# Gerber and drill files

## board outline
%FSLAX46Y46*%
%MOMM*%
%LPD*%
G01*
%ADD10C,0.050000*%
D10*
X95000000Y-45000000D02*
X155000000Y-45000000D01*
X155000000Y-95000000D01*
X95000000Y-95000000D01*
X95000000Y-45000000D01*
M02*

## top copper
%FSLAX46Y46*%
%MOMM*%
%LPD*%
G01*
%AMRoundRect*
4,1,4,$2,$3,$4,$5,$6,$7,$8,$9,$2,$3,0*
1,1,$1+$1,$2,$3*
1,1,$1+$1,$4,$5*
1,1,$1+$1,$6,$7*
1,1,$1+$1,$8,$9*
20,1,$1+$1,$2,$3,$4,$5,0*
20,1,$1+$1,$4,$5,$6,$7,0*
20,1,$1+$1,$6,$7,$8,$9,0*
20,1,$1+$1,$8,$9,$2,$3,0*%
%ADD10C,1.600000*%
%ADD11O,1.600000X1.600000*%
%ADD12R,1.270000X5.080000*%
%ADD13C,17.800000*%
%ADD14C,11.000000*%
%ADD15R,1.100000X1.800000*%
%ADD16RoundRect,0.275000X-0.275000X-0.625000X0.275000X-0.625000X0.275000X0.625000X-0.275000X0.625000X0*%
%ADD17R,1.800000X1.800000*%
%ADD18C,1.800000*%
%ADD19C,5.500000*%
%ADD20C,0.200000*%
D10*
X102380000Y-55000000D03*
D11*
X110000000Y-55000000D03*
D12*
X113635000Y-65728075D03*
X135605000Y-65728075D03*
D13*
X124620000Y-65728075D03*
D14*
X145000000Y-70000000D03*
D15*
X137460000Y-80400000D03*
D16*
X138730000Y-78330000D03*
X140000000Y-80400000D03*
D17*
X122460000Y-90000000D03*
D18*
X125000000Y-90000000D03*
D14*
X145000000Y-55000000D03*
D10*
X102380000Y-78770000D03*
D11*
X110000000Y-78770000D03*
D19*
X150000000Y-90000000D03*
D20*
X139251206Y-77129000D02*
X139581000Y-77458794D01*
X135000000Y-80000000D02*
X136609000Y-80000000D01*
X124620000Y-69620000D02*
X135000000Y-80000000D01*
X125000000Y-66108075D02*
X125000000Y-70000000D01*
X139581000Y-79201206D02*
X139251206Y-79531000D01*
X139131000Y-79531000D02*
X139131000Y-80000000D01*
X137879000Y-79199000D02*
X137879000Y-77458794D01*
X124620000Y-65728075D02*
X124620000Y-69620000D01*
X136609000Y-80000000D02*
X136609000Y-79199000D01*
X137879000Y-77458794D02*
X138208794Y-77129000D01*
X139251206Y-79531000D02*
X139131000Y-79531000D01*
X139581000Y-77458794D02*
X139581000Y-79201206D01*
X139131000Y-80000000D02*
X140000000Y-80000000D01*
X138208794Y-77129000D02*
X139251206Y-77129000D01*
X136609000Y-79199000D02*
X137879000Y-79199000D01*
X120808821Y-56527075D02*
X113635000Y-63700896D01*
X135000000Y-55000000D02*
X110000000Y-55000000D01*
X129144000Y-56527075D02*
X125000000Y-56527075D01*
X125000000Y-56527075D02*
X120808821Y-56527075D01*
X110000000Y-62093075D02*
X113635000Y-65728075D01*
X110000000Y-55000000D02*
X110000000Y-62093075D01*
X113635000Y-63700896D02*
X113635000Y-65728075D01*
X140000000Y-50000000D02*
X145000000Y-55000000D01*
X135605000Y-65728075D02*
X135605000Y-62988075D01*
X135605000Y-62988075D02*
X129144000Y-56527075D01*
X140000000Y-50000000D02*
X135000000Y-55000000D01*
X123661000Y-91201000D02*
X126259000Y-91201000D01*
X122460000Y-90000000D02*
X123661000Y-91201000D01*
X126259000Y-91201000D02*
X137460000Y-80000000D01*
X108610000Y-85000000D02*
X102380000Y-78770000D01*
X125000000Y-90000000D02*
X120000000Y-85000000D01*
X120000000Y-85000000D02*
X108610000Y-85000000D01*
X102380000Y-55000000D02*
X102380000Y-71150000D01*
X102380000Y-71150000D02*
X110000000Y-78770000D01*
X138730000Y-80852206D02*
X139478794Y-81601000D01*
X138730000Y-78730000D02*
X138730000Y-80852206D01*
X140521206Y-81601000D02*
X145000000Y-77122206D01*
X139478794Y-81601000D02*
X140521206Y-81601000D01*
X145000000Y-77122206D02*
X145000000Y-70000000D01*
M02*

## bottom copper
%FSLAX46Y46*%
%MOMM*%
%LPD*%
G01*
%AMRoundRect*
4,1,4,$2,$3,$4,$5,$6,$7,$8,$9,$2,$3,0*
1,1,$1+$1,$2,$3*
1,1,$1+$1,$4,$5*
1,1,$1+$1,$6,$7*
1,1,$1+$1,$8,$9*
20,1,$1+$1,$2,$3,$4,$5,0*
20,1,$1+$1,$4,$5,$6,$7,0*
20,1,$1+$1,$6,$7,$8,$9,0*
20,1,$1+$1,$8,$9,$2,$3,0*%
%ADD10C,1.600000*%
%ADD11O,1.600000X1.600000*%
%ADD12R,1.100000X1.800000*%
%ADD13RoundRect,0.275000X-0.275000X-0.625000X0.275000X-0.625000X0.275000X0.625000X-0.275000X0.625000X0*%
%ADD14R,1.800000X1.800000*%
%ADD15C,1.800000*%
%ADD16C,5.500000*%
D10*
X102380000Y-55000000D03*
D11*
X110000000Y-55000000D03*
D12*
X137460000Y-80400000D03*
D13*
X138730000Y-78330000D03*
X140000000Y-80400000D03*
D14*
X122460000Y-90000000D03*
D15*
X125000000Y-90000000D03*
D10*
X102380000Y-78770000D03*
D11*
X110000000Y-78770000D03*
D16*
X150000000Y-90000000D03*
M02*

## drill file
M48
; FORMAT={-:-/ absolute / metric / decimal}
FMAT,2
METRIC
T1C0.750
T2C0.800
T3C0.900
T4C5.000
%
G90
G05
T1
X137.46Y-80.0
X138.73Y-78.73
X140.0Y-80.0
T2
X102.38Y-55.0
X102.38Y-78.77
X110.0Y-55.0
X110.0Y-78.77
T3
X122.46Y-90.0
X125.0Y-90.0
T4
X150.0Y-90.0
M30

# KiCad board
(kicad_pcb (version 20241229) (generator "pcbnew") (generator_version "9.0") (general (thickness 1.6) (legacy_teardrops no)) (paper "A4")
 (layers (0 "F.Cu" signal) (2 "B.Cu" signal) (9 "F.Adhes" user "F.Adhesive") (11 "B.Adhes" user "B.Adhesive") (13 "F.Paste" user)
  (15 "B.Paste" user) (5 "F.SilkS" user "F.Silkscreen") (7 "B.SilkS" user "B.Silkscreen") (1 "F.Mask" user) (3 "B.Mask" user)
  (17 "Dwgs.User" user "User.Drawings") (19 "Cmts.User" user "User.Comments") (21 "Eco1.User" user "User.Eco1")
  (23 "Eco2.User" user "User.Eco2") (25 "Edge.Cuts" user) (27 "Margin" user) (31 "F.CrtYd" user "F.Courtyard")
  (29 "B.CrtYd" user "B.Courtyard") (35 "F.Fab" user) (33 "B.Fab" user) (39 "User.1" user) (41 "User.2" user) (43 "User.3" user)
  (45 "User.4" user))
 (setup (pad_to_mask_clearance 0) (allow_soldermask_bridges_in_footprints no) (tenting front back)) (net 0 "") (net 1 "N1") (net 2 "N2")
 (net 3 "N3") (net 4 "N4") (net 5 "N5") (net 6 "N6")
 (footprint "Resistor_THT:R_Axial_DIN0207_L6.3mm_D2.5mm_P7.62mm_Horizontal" (layer "F.Cu") (at 102.38 55)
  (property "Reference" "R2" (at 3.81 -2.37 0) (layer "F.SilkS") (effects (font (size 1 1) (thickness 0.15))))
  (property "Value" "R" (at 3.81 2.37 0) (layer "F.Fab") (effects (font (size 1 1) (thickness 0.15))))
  (pad "1" thru_hole circle (at 0 0) (size 1.6 1.6) (drill 0.8) (layers "*.Cu" "*.Mask") (remove_unused_layers no) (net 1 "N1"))
  (pad "2" thru_hole oval (at 7.62 0) (size 1.6 1.6) (drill 0.8) (layers "*.Cu" "*.Mask") (remove_unused_layers no) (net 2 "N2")))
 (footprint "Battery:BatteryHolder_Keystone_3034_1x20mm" (layer "F.Cu") (at 124.62 65.728075)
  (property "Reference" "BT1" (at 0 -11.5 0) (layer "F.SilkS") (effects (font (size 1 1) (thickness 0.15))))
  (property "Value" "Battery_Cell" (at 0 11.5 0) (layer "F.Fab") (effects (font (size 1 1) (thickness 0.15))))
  (pad "1" smd rect (at -10.985 0) (size 1.27 5.08) (layers "F.Cu" "F.Mask" "F.Paste") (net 2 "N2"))
  (pad "1" smd rect (at 10.985 0) (size 1.27 5.08) (layers "F.Cu" "F.Mask" "F.Paste") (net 2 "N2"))
  (pad "2" smd circle (at 0 0) (size 17.8 17.8) (layers "F.Cu" "F.Mask") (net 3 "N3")))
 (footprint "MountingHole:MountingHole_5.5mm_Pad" (layer "F.Cu") (at 145 70)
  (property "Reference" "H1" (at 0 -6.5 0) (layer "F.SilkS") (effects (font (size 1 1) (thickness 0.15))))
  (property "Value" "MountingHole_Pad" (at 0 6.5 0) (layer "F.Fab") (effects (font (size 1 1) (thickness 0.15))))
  (pad "1" smd circle (at 0 0) (size 11 11) (layers "F.Cu" "F.Mask" "F.Paste") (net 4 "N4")))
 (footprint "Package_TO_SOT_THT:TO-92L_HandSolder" (layer "F.Cu") (at 137.46 80)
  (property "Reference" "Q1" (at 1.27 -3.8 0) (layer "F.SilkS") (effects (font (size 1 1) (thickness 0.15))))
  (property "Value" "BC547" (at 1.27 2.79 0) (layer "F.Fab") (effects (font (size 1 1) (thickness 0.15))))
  (pad "1" thru_hole rect (at 0 0) (size 1.1 1.8) (drill 0.75 (offset 0 0.4)) (layers "*.Cu" "*.Mask") (remove_unused_layers no)
   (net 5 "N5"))
  (pad "2" thru_hole roundrect (at 1.27 -1.27) (size 1.1 1.8) (drill 0.75 (offset 0 -0.4)) (layers "*.Cu" "*.Mask")
   (remove_unused_layers no) (roundrect_rratio 0.25) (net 4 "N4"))
  (pad "3" thru_hole roundrect (at 2.54 0) (size 1.1 1.8) (drill 0.75 (offset 0 0.4)) (layers "*.Cu" "*.Mask") (remove_unused_layers no)
   (roundrect_rratio 0.25) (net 3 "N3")))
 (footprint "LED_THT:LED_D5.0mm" (layer "F.Cu") (at 122.46 90)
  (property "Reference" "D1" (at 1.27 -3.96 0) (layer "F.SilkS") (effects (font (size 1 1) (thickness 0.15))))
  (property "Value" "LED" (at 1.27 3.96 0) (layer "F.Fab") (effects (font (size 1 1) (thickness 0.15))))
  (pad "1" thru_hole rect (at 0 0) (size 1.8 1.8) (drill 0.9) (layers "*.Cu" "*.Mask") (remove_unused_layers no) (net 5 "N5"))
  (pad "2" thru_hole circle (at 2.54 0) (size 1.8 1.8) (drill 0.9) (layers "*.Cu" "*.Mask") (remove_unused_layers no) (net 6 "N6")))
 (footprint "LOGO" (layer "F.Cu") (at 140 90)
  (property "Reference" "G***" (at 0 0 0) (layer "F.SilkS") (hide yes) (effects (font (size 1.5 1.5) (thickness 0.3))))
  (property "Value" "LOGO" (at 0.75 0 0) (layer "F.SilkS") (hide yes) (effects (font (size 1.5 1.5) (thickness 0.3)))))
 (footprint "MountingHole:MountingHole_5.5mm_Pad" (layer "F.Cu") (at 145 55)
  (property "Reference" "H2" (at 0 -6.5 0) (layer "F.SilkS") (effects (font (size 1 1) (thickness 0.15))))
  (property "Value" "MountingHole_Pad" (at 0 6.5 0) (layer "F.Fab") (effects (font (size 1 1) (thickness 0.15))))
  (pad "1" smd circle (at 0 0) (size 11 11) (layers "F.Cu" "F.Mask" "F.Paste") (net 2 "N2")))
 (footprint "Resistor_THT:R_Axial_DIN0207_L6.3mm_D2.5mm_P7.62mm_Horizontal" (layer "F.Cu") (at 102.38 78.77)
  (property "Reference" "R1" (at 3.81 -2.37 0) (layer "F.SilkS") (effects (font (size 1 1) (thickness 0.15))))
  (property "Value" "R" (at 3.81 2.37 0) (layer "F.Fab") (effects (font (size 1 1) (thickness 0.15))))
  (pad "1" thru_hole circle (at 0 0) (size 1.6 1.6) (drill 0.8) (layers "*.Cu" "*.Mask") (remove_unused_layers no) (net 6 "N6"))
  (pad "2" thru_hole oval (at 7.62 0) (size 1.6 1.6) (drill 0.8) (layers "*.Cu" "*.Mask") (remove_unused_layers no) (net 1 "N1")))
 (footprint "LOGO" (layer "F.Cu") (at 101.514924 88.465482)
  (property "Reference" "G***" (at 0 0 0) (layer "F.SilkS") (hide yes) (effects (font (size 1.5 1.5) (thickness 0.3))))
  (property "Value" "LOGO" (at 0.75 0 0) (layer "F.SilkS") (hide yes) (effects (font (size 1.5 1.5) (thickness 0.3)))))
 (gr_poly (pts (xy 95 45) (xy 155 45) (xy 155 95) (xy 95 95)) (stroke (width 0.05) (type solid)) (fill no) (locked yes) (layer "Edge.Cuts"))
 (via (at 150 90) (size 5.5) (drill 5) (layers "F.Cu" "B.Cu") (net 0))
 (segment (start 139.251206 77.129) (end 139.581 77.458794) (width 0.2) (layer "F.Cu") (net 3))
 (segment (start 135 80) (end 136.609 80) (width 0.2) (layer "F.Cu") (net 3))
 (segment (start 124.62 69.62) (end 135 80) (width 0.2) (layer "F.Cu") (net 3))
 (segment (start 125 66.108075) (end 125 70) (width 0.2) (layer "F.Cu") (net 3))
 (segment (start 139.581 79.201206) (end 139.251206 79.531) (width 0.2) (layer "F.Cu") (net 3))
 (segment (start 139.131 79.531) (end 139.131 80) (width 0.2) (layer "F.Cu") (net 3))
 (segment (start 137.879 79.199) (end 137.879 77.458794) (width 0.2) (layer "F.Cu") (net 3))
 (segment (start 124.62 65.728075) (end 124.62 69.62) (width 0.2) (layer "F.Cu") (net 3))
 (segment (start 136.609 80) (end 136.609 79.199) (width 0.2) (layer "F.Cu") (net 3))
 (segment (start 137.879 77.458794) (end 138.208794 77.129) (width 0.2) (layer "F.Cu") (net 3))
 (segment (start 139.251206 79.531) (end 139.131 79.531) (width 0.2) (layer "F.Cu") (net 3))
 (segment (start 139.581 77.458794) (end 139.581 79.201206) (width 0.2) (layer "F.Cu") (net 3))
 (segment (start 139.131 80) (end 140 80) (width 0.2) (layer "F.Cu") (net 3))
 (segment (start 138.208794 77.129) (end 139.251206 77.129) (width 0.2) (layer "F.Cu") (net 3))
 (segment (start 136.609 79.199) (end 137.879 79.199) (width 0.2) (layer "F.Cu") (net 3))
 (segment (start 120.808821 56.527075) (end 113.635 63.700896) (width 0.2) (layer "F.Cu") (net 2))
 (segment (start 135 55) (end 110 55) (width 0.2) (layer "F.Cu") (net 2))
 (segment (start 129.144 56.527075) (end 125 56.527075) (width 0.2) (layer "F.Cu") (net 2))
 (segment (start 125 56.527075) (end 120.808821 56.527075) (width 0.2) (layer "F.Cu") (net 2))
 (segment (start 110 62.093075) (end 113.635 65.728075) (width 0.2) (layer "F.Cu") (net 2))
 (segment (start 110 55) (end 110 62.093075) (width 0.2) (layer "F.Cu") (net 2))
 (segment (start 113.635 63.700896) (end 113.635 65.728075) (width 0.2) (layer "F.Cu") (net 2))
 (segment (start 140 50) (end 145 55) (width 0.2) (layer "F.Cu") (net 2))
 (segment (start 135.605 65.728075) (end 135.605 62.988075) (width 0.2) (layer "F.Cu") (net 2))
 (segment (start 135.605 62.988075) (end 129.144 56.527075) (width 0.2) (layer "F.Cu") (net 2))
 (segment (start 140 50) (end 135 55) (width 0.2) (layer "F.Cu") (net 2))
 (segment (start 123.661 91.201) (end 126.259 91.201) (width 0.2) (layer "F.Cu") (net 5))
 (segment (start 122.46 90) (end 123.661 91.201) (width 0.2) (layer "F.Cu") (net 5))
 (segment (start 126.259 91.201) (end 137.46 80) (width 0.2) (layer "F.Cu") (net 5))
 (segment (start 108.61 85) (end 102.38 78.77) (width 0.2) (layer "F.Cu") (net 6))
 (segment (start 125 90) (end 120 85) (width 0.2) (layer "F.Cu") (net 6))
 (segment (start 120 85) (end 108.61 85) (width 0.2) (layer "F.Cu") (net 6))
 (segment (start 102.38 55) (end 102.38 71.15) (width 0.2) (layer "F.Cu") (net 1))
 (segment (start 102.38 71.15) (end 110 78.77) (width 0.2) (layer "F.Cu") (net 1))
 (segment (start 138.73 80.852206) (end 139.478794 81.601) (width 0.2) (layer "F.Cu") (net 4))
 (segment (start 138.73 78.73) (end 138.73 80.852206) (width 0.2) (layer "F.Cu") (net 4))
 (segment (start 140.521206 81.601) (end 145 77.122206) (width 0.2) (layer "F.Cu") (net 4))
 (segment (start 139.478794 81.601) (end 140.521206 81.601) (width 0.2) (layer "F.Cu") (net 4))
 (segment (start 145 77.122206) (end 145 70) (width 0.2) (layer "F.Cu") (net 4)))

